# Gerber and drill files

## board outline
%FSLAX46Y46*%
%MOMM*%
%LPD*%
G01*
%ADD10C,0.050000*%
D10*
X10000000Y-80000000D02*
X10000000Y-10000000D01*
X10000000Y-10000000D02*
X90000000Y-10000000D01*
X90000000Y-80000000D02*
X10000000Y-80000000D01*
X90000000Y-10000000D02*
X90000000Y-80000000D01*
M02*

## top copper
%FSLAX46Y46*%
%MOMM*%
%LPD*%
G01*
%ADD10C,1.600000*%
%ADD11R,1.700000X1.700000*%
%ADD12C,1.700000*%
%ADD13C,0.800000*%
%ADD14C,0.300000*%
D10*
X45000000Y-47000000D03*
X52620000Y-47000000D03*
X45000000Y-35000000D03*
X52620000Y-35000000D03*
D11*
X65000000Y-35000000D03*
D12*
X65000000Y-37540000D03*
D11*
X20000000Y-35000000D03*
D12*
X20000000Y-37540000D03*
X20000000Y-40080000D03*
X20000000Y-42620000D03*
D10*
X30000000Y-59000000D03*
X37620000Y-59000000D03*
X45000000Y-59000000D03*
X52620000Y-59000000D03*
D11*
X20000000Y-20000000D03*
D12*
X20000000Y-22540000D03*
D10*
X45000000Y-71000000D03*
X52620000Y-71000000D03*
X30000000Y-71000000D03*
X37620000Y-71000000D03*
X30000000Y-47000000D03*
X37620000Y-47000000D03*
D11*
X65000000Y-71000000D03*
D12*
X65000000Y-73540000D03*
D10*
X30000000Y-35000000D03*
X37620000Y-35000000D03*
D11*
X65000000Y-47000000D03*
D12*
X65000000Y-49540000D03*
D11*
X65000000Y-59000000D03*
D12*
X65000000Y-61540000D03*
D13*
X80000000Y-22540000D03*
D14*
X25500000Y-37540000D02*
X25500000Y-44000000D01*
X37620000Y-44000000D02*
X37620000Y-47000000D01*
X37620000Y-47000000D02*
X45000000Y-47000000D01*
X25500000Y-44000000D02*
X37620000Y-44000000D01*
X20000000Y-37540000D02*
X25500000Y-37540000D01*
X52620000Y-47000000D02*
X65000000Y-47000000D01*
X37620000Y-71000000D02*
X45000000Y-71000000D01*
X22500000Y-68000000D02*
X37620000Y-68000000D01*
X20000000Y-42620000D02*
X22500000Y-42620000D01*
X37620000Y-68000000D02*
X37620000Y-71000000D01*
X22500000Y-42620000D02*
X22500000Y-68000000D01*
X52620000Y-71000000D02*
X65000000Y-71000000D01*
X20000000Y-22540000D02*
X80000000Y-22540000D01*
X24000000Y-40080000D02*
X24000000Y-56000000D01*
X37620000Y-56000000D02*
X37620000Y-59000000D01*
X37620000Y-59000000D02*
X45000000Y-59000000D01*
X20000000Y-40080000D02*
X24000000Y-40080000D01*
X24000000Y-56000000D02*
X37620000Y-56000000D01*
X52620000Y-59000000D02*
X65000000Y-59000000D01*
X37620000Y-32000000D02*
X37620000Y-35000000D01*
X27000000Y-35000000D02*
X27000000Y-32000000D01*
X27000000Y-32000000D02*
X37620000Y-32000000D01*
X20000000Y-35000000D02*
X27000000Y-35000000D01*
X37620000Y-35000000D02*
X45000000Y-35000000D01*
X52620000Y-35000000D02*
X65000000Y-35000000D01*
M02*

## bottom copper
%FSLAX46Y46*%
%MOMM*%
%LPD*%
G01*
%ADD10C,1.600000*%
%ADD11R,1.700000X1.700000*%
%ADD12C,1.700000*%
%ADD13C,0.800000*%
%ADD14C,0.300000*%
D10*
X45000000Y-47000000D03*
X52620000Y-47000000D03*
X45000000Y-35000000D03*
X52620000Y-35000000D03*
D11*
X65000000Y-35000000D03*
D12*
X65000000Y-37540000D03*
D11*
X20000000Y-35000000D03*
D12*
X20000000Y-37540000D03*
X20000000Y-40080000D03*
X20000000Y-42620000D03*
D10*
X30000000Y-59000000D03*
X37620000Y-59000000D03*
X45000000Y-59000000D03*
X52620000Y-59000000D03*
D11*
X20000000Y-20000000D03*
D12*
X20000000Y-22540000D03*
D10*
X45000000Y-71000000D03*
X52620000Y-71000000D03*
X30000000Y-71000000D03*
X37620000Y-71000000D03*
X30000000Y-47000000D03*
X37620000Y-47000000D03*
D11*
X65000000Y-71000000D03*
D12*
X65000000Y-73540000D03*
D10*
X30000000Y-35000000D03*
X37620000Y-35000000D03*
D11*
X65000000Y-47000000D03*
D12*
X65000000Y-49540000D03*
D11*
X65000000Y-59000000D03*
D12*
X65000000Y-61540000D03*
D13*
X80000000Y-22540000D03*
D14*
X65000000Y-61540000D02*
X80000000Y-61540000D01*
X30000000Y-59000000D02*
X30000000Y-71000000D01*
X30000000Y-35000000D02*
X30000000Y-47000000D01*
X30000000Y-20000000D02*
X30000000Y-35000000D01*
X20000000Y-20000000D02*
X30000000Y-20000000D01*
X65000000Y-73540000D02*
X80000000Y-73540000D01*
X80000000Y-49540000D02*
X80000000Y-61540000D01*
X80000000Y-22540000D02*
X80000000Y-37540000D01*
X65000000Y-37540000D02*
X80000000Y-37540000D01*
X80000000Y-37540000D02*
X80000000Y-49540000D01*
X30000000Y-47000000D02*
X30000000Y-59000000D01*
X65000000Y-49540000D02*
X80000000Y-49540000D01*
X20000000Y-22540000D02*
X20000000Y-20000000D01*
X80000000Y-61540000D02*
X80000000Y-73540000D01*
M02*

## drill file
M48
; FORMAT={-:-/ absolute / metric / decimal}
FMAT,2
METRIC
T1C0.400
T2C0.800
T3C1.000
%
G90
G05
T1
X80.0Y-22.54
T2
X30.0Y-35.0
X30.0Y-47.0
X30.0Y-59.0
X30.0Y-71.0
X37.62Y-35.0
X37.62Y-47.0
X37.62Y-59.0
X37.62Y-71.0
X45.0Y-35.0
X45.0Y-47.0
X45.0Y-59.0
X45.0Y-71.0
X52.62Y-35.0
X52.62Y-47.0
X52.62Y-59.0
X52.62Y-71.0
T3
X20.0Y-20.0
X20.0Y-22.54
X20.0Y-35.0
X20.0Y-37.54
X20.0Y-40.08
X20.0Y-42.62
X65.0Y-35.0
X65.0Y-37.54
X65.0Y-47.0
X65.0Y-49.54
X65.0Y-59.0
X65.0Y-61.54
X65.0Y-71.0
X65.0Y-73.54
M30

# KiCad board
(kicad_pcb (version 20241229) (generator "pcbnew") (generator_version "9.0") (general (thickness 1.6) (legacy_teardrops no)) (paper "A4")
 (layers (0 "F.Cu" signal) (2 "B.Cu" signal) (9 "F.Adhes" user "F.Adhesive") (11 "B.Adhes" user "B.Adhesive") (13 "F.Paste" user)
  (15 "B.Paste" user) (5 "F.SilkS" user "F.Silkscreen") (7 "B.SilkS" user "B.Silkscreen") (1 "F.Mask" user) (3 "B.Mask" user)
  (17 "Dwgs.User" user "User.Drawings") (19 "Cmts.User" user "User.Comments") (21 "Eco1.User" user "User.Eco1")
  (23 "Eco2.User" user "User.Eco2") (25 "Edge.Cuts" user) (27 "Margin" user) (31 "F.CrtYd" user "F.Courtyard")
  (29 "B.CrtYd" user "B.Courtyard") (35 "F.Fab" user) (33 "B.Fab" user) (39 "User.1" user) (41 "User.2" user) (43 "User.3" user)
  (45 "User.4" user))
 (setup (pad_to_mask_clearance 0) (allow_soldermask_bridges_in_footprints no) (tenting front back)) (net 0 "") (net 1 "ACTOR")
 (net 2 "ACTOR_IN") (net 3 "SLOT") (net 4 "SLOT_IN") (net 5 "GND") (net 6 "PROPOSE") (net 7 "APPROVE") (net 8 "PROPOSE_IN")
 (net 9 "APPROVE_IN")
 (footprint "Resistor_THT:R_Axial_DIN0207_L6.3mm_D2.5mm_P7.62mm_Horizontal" (layer "F.Cu") (at 45 47)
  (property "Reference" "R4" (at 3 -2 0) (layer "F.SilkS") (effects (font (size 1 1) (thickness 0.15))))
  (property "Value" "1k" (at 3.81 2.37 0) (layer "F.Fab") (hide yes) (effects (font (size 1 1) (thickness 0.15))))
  (pad "1" thru_hole circle (at 0 0) (size 1.6 1.6) (drill 0.8) (layers "*.Cu" "*.Mask") (remove_unused_layers no) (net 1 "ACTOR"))
  (pad "2" thru_hole circle (at 7.62 0) (size 1.6 1.6) (drill 0.8) (layers "*.Cu" "*.Mask") (remove_unused_layers no) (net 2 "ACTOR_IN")))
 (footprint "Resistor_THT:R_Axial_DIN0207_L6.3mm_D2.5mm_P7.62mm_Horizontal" (layer "F.Cu") (at 45 35)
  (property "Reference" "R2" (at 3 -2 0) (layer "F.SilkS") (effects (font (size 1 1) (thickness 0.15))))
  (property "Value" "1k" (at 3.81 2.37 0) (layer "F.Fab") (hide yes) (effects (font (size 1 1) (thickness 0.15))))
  (pad "1" thru_hole circle (at 0 0) (size 1.6 1.6) (drill 0.8) (layers "*.Cu" "*.Mask") (remove_unused_layers no) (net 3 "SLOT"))
  (pad "2" thru_hole circle (at 7.62 0) (size 1.6 1.6) (drill 0.8) (layers "*.Cu" "*.Mask") (remove_unused_layers no) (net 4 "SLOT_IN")))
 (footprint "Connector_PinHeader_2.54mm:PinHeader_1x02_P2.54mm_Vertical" (layer "F.Cu") (at 65 35)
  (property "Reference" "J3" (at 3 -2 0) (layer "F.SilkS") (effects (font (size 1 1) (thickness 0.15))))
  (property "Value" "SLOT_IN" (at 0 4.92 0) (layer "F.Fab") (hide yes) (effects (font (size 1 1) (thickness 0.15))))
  (pad "1" thru_hole rect (at 0 0) (size 1.7 1.7) (drill 1) (layers "*.Cu" "*.Mask") (remove_unused_layers no) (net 4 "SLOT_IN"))
  (pad "2" thru_hole circle (at 0 2.54) (size 1.7 1.7) (drill 1) (layers "*.Cu" "*.Mask") (remove_unused_layers no) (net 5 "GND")))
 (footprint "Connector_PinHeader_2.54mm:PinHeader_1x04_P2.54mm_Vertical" (layer "F.Cu") (at 20 35)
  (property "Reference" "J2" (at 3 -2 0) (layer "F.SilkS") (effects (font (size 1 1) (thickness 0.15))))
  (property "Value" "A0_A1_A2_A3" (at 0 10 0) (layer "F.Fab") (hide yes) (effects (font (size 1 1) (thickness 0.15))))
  (pad "1" thru_hole rect (at 0 0) (size 1.7 1.7) (drill 1) (layers "*.Cu" "*.Mask") (remove_unused_layers no) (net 3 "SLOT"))
  (pad "2" thru_hole circle (at 0 2.54) (size 1.7 1.7) (drill 1) (layers "*.Cu" "*.Mask") (remove_unused_layers no) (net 1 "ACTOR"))
  (pad "3" thru_hole circle (at 0 5.08) (size 1.7 1.7) (drill 1) (layers "*.Cu" "*.Mask") (remove_unused_layers no) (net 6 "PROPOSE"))
  (pad "4" thru_hole circle (at 0 7.62) (size 1.7 1.7) (drill 1) (layers "*.Cu" "*.Mask") (remove_unused_layers no) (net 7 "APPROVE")))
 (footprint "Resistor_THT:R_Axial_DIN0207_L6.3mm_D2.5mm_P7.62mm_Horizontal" (layer "F.Cu") (at 30 59)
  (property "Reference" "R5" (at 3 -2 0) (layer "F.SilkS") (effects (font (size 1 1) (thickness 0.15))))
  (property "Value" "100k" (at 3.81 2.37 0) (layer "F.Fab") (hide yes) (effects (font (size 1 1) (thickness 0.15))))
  (pad "1" thru_hole circle (at 0 0) (size 1.6 1.6) (drill 0.8) (layers "*.Cu" "*.Mask") (remove_unused_layers no) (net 5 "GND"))
  (pad "2" thru_hole circle (at 7.62 0) (size 1.6 1.6) (drill 0.8) (layers "*.Cu" "*.Mask") (remove_unused_layers no) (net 6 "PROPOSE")))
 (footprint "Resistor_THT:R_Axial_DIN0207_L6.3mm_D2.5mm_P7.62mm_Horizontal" (layer "F.Cu") (at 45 59)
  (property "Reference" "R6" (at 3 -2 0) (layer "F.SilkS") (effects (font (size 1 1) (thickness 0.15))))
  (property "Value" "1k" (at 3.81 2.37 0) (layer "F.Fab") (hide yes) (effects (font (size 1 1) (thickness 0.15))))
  (pad "1" thru_hole circle (at 0 0) (size 1.6 1.6) (drill 0.8) (layers "*.Cu" "*.Mask") (remove_unused_layers no) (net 6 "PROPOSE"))
  (pad "2" thru_hole circle (at 7.62 0) (size 1.6 1.6) (drill 0.8) (layers "*.Cu" "*.Mask") (remove_unused_layers no) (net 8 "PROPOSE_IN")))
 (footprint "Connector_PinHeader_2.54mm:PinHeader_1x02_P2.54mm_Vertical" (layer "F.Cu") (at 20 20)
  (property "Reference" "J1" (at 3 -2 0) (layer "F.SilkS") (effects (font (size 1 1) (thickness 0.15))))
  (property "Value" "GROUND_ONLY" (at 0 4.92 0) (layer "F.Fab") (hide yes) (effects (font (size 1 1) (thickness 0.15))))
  (pad "1" thru_hole rect (at 0 0) (size 1.7 1.7) (drill 1) (layers "*.Cu" "*.Mask") (remove_unused_layers no) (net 5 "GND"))
  (pad "2" thru_hole circle (at 0 2.54) (size 1.7 1.7) (drill 1) (layers "*.Cu" "*.Mask") (remove_unused_layers no) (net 5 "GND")))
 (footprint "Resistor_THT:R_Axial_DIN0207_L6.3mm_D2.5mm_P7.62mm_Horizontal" (layer "F.Cu") (at 45 71)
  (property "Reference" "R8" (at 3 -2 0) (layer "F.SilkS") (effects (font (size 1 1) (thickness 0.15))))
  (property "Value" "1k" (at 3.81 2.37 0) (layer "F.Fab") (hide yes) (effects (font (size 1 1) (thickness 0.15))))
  (pad "1" thru_hole circle (at 0 0) (size 1.6 1.6) (drill 0.8) (layers "*.Cu" "*.Mask") (remove_unused_layers no) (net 7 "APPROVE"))
  (pad "2" thru_hole circle (at 7.62 0) (size 1.6 1.6) (drill 0.8) (layers "*.Cu" "*.Mask") (remove_unused_layers no) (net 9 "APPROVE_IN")))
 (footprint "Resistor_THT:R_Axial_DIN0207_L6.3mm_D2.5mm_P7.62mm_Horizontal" (layer "F.Cu") (at 30 71)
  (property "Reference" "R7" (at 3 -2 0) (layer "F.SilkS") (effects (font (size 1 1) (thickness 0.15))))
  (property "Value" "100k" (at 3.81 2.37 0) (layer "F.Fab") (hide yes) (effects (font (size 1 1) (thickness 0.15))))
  (pad "1" thru_hole circle (at 0 0) (size 1.6 1.6) (drill 0.8) (layers "*.Cu" "*.Mask") (remove_unused_layers no) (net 5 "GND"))
  (pad "2" thru_hole circle (at 7.62 0) (size 1.6 1.6) (drill 0.8) (layers "*.Cu" "*.Mask") (remove_unused_layers no) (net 7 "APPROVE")))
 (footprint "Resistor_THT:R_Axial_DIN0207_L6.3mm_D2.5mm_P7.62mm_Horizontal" (layer "F.Cu") (at 30 47)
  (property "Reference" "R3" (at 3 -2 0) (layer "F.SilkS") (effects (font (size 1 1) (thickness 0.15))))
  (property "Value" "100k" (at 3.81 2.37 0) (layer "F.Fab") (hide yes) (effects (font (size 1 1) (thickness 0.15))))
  (pad "1" thru_hole circle (at 0 0) (size 1.6 1.6) (drill 0.8) (layers "*.Cu" "*.Mask") (remove_unused_layers no) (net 5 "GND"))
  (pad "2" thru_hole circle (at 7.62 0) (size 1.6 1.6) (drill 0.8) (layers "*.Cu" "*.Mask") (remove_unused_layers no) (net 1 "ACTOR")))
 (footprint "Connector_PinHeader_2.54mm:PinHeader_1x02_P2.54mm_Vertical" (layer "F.Cu") (at 65 71)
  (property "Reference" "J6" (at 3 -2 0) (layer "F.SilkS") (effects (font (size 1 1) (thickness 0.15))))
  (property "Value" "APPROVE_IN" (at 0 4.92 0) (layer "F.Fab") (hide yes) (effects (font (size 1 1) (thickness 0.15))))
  (pad "1" thru_hole rect (at 0 0) (size 1.7 1.7) (drill 1) (layers "*.Cu" "*.Mask") (remove_unused_layers no) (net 9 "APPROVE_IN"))
  (pad "2" thru_hole circle (at 0 2.54) (size 1.7 1.7) (drill 1) (layers "*.Cu" "*.Mask") (remove_unused_layers no) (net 5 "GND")))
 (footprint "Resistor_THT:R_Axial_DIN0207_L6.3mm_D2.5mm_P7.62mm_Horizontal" (layer "F.Cu") (at 30 35)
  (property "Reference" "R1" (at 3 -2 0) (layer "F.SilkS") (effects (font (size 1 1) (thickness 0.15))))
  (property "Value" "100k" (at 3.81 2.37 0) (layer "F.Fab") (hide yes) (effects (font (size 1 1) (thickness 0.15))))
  (pad "1" thru_hole circle (at 0 0) (size 1.6 1.6) (drill 0.8) (layers "*.Cu" "*.Mask") (remove_unused_layers no) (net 5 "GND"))
  (pad "2" thru_hole circle (at 7.62 0) (size 1.6 1.6) (drill 0.8) (layers "*.Cu" "*.Mask") (remove_unused_layers no) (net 3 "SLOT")))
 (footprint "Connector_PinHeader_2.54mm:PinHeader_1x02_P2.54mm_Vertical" (layer "F.Cu") (at 65 47)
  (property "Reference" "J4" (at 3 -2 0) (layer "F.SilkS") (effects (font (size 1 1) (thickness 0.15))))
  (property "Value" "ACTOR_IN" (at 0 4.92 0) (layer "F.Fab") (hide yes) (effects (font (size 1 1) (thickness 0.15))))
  (pad "1" thru_hole rect (at 0 0) (size 1.7 1.7) (drill 1) (layers "*.Cu" "*.Mask") (remove_unused_layers no) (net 2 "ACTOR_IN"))
  (pad "2" thru_hole circle (at 0 2.54) (size 1.7 1.7) (drill 1) (layers "*.Cu" "*.Mask") (remove_unused_layers no) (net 5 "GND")))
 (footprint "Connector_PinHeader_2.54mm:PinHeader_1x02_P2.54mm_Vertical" (layer "F.Cu") (at 65 59)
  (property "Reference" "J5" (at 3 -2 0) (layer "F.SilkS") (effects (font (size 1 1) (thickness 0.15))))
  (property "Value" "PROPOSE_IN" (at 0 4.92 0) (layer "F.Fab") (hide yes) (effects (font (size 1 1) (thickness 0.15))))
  (pad "1" thru_hole rect (at 0 0) (size 1.7 1.7) (drill 1) (layers "*.Cu" "*.Mask") (remove_unused_layers no) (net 8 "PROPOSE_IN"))
  (pad "2" thru_hole circle (at 0 2.54) (size 1.7 1.7) (drill 1) (layers "*.Cu" "*.Mask") (remove_unused_layers no) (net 5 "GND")))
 (gr_line (start 10 80) (end 10 10) (stroke (width 0.05) (type default)) (layer "Edge.Cuts"))
 (gr_line (start 10 10) (end 90 10) (stroke (width 0.05) (type default)) (layer "Edge.Cuts"))
 (gr_line (start 90 80) (end 10 80) (stroke (width 0.05) (type default)) (layer "Edge.Cuts"))
 (gr_line (start 90 10) (end 90 80) (stroke (width 0.05) (type default)) (layer "Edge.Cuts"))
 (segment (start 25.5 37.54) (end 25.5 44) (width 0.3) (layer "F.Cu") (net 1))
 (segment (start 37.62 44) (end 37.62 47) (width 0.3) (layer "F.Cu") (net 1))
 (segment (start 37.62 47) (end 45 47) (width 0.3) (layer "F.Cu") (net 1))
 (segment (start 25.5 44) (end 37.62 44) (width 0.3) (layer "F.Cu") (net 1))
 (segment (start 20 37.54) (end 25.5 37.54) (width 0.3) (layer "F.Cu") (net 1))
 (segment (start 52.62 47) (end 65 47) (width 0.3) (layer "F.Cu") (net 2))
 (segment (start 37.62 71) (end 45 71) (width 0.3) (layer "F.Cu") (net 7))
 (segment (start 22.5 68) (end 37.62 68) (width 0.3) (layer "F.Cu") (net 7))
 (segment (start 20 42.62) (end 22.5 42.62) (width 0.3) (layer "F.Cu") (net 7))
 (segment (start 37.62 68) (end 37.62 71) (width 0.3) (layer "F.Cu") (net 7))
 (segment (start 22.5 42.62) (end 22.5 68) (width 0.3) (layer "F.Cu") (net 7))
 (segment (start 52.62 71) (end 65 71) (width 0.3) (layer "F.Cu") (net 9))
 (segment (start 20 22.54) (end 80 22.54) (width 0.3) (layer "F.Cu") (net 5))
 (via (at 80 22.54) (size 0.8) (drill 0.4) (layers "F.Cu" "B.Cu") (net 5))
 (segment (start 65 61.54) (end 80 61.54) (width 0.3) (layer "B.Cu") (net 5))
 (segment (start 30 59) (end 30 71) (width 0.3) (layer "B.Cu") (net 5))
 (segment (start 30 35) (end 30 47) (width 0.3) (layer "B.Cu") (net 5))
 (segment (start 30 20) (end 30 35) (width 0.3) (layer "B.Cu") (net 5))
 (segment (start 20 20) (end 30 20) (width 0.3) (layer "B.Cu") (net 5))
 (segment (start 65 73.54) (end 80 73.54) (width 0.3) (layer "B.Cu") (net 5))
 (segment (start 80 49.54) (end 80 61.54) (width 0.3) (layer "B.Cu") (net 5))
 (segment (start 80 22.54) (end 80 37.54) (width 0.3) (layer "B.Cu") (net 5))
 (segment (start 65 37.54) (end 80 37.54) (width 0.3) (layer "B.Cu") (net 5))
 (segment (start 80 37.54) (end 80 49.54) (width 0.3) (layer "B.Cu") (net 5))
 (segment (start 30 47) (end 30 59) (width 0.3) (layer "B.Cu") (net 5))
 (segment (start 65 49.54) (end 80 49.54) (width 0.3) (layer "B.Cu") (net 5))
 (segment (start 20 22.54) (end 20 20) (width 0.3) (layer "B.Cu") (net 5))
 (segment (start 80 61.54) (end 80 73.54) (width 0.3) (layer "B.Cu") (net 5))
 (segment (start 24 40.08) (end 24 56) (width 0.3) (layer "F.Cu") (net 6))
 (segment (start 37.62 56) (end 37.62 59) (width 0.3) (layer "F.Cu") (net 6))
 (segment (start 37.62 59) (end 45 59) (width 0.3) (layer "F.Cu") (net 6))
 (segment (start 20 40.08) (end 24 40.08) (width 0.3) (layer "F.Cu") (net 6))
 (segment (start 24 56) (end 37.62 56) (width 0.3) (layer "F.Cu") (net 6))
 (segment (start 52.62 59) (end 65 59) (width 0.3) (layer "F.Cu") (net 8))
 (segment (start 37.62 32) (end 37.62 35) (width 0.3) (layer "F.Cu") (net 3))
 (segment (start 27 35) (end 27 32) (width 0.3) (layer "F.Cu") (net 3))
 (segment (start 27 32) (end 37.62 32) (width 0.3) (layer "F.Cu") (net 3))
 (segment (start 20 35) (end 27 35) (width 0.3) (layer "F.Cu") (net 3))
 (segment (start 37.62 35) (end 45 35) (width 0.3) (layer "F.Cu") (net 3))
 (segment (start 52.62 35) (end 65 35) (width 0.3) (layer "F.Cu") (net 4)))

